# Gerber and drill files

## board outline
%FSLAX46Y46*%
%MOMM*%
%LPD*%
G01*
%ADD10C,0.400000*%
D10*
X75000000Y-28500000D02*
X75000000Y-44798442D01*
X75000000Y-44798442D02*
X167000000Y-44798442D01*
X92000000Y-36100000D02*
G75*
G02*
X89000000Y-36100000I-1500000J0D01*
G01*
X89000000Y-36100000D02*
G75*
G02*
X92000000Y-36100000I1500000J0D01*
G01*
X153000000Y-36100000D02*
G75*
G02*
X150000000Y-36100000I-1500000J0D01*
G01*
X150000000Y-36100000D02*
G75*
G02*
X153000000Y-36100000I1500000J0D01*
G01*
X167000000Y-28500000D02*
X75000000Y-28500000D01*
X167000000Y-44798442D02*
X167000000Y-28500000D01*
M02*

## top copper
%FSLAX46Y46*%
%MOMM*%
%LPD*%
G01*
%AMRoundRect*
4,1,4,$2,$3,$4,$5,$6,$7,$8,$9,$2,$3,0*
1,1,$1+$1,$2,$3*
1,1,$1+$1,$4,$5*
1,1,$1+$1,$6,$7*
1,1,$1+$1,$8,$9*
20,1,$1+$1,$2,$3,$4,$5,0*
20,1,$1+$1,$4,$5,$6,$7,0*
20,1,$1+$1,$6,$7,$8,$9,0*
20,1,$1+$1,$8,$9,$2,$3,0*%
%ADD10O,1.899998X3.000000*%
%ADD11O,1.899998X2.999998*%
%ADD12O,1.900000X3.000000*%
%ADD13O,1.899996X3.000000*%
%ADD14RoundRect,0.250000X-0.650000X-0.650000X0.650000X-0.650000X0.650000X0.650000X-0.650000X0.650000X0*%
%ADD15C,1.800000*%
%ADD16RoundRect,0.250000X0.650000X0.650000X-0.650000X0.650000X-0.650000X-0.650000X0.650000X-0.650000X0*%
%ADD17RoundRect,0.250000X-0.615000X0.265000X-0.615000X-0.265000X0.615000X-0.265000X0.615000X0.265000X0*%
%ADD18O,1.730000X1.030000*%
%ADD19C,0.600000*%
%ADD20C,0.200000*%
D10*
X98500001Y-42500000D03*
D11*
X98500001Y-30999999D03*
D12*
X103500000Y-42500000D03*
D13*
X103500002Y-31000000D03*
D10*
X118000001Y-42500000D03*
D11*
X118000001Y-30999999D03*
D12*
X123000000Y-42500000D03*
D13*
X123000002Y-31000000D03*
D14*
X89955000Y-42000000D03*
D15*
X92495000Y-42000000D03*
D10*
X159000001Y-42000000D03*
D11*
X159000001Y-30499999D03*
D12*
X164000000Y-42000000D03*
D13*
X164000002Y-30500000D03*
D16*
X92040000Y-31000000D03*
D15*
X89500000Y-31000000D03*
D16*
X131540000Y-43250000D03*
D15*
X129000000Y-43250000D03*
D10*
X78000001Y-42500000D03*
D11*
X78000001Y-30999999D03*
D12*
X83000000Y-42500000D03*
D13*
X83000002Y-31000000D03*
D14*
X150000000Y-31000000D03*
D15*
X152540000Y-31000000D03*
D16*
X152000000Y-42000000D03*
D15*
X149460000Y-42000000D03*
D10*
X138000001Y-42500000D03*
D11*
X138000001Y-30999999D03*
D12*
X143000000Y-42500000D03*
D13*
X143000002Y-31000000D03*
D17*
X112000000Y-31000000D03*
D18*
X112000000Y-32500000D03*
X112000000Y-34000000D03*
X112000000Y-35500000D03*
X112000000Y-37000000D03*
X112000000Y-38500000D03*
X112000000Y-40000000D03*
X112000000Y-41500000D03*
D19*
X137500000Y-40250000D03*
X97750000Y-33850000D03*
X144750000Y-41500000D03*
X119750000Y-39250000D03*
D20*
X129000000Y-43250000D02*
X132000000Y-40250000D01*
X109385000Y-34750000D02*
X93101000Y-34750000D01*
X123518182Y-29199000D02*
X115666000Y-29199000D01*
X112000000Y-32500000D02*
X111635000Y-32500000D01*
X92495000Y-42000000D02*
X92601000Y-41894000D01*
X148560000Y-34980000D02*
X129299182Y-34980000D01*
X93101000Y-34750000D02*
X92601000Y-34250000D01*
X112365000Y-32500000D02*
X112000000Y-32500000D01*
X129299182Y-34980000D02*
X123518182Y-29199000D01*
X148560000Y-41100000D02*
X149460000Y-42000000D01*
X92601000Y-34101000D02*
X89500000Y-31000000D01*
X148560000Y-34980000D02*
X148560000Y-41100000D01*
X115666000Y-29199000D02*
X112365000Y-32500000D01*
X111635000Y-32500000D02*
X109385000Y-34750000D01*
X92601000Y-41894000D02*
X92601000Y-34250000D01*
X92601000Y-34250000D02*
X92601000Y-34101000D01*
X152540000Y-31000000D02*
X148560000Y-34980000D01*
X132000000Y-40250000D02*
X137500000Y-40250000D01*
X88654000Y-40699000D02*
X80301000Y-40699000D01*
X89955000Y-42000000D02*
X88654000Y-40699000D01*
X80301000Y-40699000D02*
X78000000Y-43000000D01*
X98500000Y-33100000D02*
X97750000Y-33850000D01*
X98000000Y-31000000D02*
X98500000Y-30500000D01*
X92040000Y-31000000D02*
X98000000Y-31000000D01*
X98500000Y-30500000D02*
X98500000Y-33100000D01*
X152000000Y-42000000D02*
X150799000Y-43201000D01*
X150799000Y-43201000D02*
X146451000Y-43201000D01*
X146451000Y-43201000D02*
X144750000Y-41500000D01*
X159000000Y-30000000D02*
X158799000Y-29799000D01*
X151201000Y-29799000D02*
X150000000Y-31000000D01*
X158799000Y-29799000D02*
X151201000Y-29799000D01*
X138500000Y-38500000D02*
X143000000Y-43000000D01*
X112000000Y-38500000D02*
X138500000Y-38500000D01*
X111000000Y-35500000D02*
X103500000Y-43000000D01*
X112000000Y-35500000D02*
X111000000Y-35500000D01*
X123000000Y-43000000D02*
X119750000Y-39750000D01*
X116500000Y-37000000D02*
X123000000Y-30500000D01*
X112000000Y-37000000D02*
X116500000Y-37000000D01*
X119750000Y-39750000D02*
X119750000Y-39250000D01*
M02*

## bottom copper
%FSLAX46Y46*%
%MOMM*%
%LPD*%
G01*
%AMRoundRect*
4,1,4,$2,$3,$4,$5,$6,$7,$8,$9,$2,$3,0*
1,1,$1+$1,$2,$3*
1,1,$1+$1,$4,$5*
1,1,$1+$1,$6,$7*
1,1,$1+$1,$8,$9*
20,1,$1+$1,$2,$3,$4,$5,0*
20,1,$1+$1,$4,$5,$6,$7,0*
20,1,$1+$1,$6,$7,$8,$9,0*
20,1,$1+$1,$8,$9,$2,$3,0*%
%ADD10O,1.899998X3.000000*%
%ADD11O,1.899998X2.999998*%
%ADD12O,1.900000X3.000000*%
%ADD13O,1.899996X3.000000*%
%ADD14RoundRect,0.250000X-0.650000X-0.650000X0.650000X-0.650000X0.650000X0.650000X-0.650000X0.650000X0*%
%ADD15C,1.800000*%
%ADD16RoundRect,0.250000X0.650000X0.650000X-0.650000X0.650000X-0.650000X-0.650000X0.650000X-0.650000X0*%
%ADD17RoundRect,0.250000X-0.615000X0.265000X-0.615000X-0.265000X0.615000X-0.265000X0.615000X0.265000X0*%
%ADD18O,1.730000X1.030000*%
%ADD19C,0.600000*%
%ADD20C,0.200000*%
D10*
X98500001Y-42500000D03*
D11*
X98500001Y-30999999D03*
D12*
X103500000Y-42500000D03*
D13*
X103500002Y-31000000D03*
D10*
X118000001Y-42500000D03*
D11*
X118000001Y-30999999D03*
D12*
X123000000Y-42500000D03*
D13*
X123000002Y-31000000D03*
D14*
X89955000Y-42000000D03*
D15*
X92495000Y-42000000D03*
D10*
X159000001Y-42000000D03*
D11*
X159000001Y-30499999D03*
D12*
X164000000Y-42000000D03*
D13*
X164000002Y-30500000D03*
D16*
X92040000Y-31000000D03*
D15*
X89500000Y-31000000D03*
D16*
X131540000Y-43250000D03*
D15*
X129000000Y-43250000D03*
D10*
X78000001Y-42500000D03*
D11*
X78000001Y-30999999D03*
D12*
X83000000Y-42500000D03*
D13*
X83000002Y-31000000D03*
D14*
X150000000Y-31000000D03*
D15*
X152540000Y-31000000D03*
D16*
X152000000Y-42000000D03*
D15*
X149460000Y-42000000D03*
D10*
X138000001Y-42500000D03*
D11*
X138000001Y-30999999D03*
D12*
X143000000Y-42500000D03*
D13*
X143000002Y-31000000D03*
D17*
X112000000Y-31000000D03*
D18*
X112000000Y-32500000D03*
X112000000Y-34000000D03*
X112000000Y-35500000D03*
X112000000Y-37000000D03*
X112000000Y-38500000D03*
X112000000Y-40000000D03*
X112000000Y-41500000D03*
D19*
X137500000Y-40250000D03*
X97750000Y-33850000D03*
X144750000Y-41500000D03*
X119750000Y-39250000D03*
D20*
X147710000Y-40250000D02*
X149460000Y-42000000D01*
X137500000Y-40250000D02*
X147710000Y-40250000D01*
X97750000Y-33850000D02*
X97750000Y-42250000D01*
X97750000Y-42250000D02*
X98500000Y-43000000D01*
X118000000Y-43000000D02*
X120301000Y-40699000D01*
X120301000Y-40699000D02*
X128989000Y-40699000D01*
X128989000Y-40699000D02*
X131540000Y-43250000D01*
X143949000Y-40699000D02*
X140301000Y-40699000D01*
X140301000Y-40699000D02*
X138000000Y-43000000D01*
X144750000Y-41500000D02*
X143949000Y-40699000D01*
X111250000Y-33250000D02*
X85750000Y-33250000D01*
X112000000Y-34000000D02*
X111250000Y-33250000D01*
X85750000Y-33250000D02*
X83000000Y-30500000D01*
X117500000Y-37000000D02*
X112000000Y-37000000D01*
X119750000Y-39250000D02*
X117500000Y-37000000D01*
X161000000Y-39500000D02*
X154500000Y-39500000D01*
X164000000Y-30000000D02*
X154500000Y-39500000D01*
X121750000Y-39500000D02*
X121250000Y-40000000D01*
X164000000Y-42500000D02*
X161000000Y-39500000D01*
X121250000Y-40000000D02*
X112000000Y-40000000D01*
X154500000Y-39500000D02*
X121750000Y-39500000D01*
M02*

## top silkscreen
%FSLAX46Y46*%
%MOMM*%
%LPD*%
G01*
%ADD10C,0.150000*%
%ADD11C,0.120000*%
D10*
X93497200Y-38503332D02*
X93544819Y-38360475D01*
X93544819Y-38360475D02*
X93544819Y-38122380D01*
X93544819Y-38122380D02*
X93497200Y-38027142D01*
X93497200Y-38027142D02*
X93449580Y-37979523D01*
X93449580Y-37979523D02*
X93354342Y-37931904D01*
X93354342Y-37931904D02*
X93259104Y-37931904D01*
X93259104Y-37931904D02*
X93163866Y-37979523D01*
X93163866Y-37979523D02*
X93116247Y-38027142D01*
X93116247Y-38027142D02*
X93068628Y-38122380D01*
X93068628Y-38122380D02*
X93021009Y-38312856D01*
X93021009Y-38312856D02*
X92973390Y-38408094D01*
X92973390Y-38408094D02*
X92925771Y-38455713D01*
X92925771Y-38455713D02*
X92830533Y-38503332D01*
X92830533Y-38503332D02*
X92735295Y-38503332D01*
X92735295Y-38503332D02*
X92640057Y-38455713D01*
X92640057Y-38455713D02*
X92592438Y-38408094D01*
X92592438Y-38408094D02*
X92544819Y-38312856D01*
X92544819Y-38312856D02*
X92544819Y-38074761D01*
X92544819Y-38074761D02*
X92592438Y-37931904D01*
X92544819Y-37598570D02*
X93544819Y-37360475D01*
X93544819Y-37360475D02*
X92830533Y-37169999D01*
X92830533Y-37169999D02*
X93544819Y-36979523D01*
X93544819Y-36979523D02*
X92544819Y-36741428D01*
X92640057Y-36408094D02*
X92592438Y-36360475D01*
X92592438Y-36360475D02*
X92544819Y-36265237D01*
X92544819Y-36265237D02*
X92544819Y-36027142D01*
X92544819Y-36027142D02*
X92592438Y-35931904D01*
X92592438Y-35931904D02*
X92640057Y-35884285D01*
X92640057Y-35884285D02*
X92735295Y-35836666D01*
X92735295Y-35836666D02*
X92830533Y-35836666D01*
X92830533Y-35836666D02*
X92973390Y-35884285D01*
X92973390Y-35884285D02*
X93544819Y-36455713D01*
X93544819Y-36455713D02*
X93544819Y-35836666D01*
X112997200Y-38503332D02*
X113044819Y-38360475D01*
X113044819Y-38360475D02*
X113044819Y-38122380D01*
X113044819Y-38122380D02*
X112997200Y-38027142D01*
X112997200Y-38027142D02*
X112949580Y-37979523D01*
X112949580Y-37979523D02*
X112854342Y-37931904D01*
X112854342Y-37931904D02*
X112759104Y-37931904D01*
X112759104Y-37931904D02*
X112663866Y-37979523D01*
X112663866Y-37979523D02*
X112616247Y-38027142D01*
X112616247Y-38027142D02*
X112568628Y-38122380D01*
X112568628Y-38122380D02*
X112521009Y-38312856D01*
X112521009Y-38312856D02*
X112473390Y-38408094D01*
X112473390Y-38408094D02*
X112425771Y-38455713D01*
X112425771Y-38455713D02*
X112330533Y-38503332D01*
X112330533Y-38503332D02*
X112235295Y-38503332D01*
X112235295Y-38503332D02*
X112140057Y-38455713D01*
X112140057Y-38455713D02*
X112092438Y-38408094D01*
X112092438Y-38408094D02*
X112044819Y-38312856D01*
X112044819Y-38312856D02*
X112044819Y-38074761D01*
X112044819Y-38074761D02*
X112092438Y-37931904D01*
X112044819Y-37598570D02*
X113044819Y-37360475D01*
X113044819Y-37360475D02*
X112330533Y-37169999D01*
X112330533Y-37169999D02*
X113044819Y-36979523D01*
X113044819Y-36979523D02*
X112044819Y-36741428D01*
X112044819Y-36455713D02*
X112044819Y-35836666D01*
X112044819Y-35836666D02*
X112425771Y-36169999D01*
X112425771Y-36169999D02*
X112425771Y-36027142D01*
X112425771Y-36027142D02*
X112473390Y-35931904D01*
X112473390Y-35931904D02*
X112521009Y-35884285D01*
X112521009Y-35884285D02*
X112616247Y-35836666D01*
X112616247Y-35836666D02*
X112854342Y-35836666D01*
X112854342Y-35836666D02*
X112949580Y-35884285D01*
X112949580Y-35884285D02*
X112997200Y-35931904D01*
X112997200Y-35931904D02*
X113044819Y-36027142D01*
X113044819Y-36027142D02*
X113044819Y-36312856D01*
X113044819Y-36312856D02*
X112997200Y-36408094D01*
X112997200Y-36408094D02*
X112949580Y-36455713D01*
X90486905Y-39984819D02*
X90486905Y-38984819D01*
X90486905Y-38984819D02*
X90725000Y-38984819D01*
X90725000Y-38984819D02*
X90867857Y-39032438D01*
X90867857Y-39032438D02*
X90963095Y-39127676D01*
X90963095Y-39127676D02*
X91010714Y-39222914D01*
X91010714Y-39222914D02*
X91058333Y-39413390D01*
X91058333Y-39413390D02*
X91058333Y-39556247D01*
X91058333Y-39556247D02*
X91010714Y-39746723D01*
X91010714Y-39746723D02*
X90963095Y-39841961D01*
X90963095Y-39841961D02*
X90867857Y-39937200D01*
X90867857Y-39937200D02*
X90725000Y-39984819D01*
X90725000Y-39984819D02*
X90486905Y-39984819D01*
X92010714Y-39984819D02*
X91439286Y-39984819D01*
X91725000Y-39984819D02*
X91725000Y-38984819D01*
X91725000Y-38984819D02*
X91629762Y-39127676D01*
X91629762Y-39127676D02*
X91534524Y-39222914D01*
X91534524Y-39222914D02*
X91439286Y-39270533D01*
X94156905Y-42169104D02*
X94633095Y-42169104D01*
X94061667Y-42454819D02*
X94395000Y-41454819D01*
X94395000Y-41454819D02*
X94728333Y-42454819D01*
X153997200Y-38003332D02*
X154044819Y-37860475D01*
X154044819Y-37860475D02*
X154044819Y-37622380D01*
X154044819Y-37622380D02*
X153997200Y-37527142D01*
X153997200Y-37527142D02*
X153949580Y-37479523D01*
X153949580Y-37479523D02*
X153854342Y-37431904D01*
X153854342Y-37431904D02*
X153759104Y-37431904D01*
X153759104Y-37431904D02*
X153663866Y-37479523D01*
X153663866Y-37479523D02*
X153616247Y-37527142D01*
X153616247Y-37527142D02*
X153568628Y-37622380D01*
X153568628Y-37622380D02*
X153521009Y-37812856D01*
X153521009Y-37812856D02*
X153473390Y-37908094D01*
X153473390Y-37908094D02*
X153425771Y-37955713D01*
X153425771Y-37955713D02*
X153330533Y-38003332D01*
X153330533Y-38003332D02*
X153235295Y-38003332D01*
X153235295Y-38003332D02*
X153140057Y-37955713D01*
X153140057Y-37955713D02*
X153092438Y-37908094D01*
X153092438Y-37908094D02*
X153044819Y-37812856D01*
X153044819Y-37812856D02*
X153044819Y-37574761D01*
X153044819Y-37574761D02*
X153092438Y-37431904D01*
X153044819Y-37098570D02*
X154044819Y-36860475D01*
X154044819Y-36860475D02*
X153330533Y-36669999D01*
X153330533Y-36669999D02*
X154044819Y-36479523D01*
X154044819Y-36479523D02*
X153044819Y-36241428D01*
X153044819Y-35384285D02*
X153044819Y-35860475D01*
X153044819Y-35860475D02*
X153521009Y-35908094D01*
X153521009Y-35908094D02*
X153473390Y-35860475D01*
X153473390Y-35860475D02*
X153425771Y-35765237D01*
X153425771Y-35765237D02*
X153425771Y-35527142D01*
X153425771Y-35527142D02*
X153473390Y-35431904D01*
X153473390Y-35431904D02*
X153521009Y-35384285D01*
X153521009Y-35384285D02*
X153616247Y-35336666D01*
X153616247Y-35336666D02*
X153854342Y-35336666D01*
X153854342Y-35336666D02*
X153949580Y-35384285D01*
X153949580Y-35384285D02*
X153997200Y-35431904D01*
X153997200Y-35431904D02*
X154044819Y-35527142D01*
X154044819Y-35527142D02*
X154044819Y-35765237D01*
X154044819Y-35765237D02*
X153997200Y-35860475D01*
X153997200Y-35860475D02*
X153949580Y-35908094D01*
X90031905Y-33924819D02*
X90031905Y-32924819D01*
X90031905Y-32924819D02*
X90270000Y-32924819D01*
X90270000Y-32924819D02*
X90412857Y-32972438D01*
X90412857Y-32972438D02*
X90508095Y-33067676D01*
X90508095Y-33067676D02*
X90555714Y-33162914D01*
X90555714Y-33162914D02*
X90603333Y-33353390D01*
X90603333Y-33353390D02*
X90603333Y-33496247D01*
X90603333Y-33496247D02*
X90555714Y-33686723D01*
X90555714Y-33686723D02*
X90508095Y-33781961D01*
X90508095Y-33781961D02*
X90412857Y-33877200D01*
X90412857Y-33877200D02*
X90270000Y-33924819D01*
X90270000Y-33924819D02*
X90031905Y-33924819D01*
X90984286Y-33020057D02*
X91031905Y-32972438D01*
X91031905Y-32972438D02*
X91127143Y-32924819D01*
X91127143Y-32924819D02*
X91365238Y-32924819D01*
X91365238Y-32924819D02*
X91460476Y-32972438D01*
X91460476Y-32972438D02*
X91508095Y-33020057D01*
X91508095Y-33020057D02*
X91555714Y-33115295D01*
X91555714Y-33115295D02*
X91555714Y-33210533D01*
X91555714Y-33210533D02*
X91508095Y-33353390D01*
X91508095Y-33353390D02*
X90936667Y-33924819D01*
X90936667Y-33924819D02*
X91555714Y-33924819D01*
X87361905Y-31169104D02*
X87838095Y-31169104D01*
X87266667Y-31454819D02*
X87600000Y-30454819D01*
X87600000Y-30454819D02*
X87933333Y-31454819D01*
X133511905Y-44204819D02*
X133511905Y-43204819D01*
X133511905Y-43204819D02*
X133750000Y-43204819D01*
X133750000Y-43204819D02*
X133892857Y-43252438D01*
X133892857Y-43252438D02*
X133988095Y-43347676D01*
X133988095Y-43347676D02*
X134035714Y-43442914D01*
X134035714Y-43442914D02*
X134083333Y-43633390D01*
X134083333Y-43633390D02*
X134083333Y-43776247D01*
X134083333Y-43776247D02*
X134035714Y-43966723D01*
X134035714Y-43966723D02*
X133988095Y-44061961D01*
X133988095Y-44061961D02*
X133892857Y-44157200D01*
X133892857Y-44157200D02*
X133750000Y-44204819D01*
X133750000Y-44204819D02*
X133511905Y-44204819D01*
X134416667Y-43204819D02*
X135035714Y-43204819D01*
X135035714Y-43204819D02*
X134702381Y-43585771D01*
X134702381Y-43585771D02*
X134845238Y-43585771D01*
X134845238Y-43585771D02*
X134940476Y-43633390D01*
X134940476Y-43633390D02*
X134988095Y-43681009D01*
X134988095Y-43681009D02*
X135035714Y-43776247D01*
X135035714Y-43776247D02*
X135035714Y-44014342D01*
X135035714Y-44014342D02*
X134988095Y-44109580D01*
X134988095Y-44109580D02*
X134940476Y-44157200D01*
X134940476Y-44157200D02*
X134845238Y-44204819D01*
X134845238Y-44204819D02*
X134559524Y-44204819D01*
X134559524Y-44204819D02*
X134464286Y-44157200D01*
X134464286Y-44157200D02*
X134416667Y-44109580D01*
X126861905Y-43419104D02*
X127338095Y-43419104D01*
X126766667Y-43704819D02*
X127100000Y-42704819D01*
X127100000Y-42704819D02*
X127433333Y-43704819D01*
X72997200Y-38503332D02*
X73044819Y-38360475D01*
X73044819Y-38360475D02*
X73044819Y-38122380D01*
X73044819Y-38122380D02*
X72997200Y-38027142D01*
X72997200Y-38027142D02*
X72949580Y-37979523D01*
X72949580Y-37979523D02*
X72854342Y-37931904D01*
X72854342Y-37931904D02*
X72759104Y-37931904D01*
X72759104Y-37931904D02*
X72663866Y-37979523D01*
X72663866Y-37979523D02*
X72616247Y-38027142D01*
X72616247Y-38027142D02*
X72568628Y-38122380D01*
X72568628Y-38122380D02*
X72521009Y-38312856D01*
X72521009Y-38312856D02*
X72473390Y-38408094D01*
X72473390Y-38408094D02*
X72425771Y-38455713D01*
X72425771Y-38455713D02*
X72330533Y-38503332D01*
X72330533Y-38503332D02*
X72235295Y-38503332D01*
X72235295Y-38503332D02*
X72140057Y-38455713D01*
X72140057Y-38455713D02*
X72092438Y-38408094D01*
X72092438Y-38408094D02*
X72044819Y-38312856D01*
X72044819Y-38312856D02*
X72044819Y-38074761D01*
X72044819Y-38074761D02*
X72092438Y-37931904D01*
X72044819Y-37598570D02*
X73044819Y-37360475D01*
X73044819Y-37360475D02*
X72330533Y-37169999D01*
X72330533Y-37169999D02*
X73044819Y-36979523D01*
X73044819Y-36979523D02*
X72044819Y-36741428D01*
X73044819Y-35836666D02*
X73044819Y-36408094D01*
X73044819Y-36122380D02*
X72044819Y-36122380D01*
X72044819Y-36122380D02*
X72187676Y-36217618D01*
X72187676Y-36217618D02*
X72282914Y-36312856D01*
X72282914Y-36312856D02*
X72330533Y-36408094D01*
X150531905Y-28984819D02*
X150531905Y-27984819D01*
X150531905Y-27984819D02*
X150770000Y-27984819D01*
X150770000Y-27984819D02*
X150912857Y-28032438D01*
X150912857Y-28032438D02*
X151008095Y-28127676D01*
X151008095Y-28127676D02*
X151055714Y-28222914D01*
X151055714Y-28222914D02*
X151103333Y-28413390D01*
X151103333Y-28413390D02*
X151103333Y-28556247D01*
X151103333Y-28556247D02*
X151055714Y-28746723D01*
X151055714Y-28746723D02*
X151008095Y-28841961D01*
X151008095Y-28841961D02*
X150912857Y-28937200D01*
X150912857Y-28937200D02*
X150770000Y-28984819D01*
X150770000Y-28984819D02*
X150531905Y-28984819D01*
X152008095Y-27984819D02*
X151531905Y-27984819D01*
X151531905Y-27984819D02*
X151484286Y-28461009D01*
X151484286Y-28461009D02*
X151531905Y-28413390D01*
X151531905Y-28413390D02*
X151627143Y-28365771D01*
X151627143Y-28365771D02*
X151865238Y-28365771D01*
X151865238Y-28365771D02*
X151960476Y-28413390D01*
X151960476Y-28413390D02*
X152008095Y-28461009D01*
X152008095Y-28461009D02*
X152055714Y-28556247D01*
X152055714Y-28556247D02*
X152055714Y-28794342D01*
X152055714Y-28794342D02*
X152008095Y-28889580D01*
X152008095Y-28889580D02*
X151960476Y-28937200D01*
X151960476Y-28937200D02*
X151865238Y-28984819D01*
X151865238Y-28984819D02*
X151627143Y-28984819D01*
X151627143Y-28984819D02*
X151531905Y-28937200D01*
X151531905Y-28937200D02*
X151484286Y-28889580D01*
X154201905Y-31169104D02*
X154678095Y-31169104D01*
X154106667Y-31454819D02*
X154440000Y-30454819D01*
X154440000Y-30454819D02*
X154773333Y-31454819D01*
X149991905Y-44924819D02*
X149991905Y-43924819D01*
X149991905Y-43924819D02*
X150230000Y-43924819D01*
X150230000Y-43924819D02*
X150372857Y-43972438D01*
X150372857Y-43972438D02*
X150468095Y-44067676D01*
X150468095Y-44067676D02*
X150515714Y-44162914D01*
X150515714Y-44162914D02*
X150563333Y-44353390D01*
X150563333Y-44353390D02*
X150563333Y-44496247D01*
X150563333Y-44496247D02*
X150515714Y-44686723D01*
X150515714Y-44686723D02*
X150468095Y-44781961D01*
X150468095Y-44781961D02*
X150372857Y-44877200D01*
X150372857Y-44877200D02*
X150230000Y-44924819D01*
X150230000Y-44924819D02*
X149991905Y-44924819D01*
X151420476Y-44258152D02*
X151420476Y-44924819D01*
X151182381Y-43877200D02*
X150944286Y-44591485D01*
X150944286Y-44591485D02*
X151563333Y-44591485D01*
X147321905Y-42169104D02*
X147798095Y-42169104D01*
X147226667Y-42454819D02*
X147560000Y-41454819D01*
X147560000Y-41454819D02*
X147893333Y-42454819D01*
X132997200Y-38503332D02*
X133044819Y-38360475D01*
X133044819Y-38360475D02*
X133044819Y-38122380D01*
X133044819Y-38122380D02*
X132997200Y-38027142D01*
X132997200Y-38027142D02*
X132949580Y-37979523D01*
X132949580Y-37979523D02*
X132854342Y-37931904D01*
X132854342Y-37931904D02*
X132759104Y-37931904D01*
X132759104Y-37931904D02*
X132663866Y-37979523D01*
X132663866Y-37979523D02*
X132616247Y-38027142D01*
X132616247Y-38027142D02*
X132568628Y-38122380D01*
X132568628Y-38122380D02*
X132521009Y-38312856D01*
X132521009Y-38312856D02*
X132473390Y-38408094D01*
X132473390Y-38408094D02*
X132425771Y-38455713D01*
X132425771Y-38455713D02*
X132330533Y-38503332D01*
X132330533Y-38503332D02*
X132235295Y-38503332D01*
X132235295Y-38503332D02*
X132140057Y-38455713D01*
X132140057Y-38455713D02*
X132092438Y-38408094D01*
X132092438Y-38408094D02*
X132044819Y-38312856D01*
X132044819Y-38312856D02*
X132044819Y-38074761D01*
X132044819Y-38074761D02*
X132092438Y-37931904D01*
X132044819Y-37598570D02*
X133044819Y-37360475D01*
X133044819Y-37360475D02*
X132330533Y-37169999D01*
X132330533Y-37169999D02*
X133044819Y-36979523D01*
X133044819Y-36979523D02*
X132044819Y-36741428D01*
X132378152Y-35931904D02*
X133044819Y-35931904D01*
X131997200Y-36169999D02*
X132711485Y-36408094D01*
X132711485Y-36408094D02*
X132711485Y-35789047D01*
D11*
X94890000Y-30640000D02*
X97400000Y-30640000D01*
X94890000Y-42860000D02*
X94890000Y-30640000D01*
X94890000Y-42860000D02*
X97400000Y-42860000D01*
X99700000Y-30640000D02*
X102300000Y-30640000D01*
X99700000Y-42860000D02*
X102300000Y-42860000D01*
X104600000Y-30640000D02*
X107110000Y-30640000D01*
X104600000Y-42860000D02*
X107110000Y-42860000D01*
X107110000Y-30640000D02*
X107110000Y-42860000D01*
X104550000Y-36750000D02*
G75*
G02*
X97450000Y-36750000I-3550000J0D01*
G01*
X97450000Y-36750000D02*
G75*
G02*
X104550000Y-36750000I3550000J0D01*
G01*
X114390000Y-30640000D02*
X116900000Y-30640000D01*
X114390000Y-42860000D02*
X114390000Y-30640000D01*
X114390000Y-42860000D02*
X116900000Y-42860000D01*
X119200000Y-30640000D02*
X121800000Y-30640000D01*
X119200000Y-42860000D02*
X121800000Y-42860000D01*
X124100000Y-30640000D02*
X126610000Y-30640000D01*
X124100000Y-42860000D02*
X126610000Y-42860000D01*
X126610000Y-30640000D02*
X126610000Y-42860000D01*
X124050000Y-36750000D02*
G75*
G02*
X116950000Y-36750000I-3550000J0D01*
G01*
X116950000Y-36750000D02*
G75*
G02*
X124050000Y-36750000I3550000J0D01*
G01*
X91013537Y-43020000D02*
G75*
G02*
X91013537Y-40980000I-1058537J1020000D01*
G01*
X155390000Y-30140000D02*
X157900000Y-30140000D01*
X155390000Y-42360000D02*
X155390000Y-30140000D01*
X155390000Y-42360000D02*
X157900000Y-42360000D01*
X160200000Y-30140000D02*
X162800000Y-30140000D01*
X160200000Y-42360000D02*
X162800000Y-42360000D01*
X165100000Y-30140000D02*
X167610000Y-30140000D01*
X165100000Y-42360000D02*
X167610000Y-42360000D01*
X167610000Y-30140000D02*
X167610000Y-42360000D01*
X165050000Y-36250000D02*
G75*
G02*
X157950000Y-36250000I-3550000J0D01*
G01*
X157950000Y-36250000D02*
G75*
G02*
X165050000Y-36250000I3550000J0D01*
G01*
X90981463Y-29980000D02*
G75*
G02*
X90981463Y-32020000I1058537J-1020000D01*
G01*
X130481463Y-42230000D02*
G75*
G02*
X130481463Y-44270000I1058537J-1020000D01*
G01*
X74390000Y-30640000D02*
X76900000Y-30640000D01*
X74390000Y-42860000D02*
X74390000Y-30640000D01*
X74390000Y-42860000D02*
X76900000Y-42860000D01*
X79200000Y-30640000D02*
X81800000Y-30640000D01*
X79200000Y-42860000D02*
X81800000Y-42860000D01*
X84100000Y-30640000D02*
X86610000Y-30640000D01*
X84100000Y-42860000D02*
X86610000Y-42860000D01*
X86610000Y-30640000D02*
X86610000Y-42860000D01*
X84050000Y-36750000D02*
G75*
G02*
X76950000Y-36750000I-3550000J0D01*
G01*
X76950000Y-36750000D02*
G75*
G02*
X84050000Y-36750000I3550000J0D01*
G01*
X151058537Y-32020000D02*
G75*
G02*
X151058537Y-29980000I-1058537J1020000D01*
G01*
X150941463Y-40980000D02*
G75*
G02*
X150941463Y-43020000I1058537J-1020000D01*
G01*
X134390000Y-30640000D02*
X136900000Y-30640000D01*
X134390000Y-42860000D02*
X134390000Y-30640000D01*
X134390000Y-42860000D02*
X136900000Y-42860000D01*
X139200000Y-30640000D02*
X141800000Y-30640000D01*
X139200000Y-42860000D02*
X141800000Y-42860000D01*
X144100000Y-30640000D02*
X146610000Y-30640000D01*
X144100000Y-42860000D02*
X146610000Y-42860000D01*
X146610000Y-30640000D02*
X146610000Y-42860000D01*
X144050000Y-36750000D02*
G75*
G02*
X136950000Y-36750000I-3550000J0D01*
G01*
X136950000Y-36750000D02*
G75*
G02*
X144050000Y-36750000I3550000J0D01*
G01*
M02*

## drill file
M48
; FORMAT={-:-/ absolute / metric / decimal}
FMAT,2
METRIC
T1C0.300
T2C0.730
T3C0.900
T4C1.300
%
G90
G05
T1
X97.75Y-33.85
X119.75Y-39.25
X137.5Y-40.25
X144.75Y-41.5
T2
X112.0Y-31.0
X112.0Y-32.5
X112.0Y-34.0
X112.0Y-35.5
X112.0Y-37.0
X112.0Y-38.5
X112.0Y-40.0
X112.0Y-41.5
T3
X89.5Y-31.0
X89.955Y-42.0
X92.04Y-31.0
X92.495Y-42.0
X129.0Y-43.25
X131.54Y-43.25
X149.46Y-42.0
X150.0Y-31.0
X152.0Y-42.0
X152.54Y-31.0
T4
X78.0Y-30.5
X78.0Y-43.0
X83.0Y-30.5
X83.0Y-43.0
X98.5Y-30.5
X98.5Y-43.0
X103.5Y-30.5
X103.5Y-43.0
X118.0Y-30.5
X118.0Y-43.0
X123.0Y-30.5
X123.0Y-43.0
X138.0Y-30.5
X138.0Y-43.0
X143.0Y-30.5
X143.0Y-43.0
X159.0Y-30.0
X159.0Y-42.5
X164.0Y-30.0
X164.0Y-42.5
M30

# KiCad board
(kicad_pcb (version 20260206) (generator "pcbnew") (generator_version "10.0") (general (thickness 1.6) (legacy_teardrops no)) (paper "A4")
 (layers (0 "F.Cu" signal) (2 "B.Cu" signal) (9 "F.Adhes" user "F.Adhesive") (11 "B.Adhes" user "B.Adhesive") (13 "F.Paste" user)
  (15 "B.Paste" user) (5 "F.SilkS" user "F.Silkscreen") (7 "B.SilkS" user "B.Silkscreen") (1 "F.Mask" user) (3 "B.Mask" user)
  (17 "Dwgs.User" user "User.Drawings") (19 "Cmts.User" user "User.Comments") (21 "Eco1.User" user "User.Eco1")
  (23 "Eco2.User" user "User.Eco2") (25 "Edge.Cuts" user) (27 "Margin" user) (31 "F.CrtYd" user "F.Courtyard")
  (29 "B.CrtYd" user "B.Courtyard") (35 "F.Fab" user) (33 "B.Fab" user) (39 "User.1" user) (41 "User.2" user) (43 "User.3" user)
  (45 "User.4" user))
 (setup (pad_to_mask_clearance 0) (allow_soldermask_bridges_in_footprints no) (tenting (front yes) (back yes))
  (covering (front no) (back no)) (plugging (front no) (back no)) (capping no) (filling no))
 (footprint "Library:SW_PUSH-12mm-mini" (layer "F.Cu") (at 98.5 43 90)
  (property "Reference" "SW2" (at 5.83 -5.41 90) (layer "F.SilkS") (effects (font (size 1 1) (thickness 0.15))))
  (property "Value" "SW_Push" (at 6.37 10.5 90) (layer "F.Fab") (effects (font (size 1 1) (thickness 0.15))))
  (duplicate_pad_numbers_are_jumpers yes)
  (fp_line (start 12.36 -3.61) (end 12.36 -1.1) (stroke (width 0.12) (type default)) (layer "F.SilkS"))
  (fp_line (start 0.14 -3.61) (end 12.36 -3.61) (stroke (width 0.12) (type default)) (layer "F.SilkS"))
  (fp_line (start 0.14 -3.61) (end 0.14 -1.1) (stroke (width 0.12) (type default)) (layer "F.SilkS"))
  (fp_line (start 12.36 1.2) (end 12.36 3.8) (stroke (width 0.12) (type default)) (layer "F.SilkS"))
  (fp_line (start 0.14 1.2) (end 0.14 3.8) (stroke (width 0.12) (type default)) (layer "F.SilkS"))
  (fp_line (start 12.36 6.1) (end 12.36 8.61) (stroke (width 0.12) (type default)) (layer "F.SilkS"))
  (fp_line (start 0.14 6.1) (end 0.14 8.61) (stroke (width 0.12) (type default)) (layer "F.SilkS"))
  (fp_line (start 12.36 8.61) (end 0.14 8.61) (stroke (width 0.12) (type default)) (layer "F.SilkS"))
  (fp_circle (center 6.25 2.5) (end 9.8 2.5) (stroke (width 0.12) (type default)) (fill no) (layer "F.SilkS"))
  (pad "1" thru_hole oval (at 0 0 90) (size 3 1.899998) (drill 1.3 (offset 0.5 0.000001)) (layers "*.Cu" "*.Mask") (remove_unused_layers no)
   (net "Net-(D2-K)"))
  (pad "1" thru_hole oval (at 12.5 0 90) (size 2.999998 1.899998) (drill 1.3 (offset -0.499999 0.000001)) (layers "*.Cu" "*.Mask")
   (remove_unused_layers no) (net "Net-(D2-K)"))
  (pad "2" thru_hole oval (at 0 5 90) (size 3 1.9) (drill 1.3 (offset 0.5 0)) (layers "*.Cu" "*.Mask") (remove_unused_layers no)
   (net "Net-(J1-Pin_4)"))
  (pad "2" thru_hole oval (at 12.5 5 90) (size 3 1.899996) (drill 1.3 (offset -0.5 0.000002)) (layers "*.Cu" "*.Mask")
   (remove_unused_layers no) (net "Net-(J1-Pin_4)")))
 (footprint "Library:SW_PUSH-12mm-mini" (layer "F.Cu") (at 118 43 90)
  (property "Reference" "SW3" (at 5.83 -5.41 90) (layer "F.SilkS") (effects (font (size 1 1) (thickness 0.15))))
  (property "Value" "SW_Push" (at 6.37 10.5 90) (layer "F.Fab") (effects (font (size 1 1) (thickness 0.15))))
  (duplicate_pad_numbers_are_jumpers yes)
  (fp_line (start 12.36 -3.61) (end 12.36 -1.1) (stroke (width 0.12) (type default)) (layer "F.SilkS"))
  (fp_line (start 0.14 -3.61) (end 12.36 -3.61) (stroke (width 0.12) (type default)) (layer "F.SilkS"))
  (fp_line (start 0.14 -3.61) (end 0.14 -1.1) (stroke (width 0.12) (type default)) (layer "F.SilkS"))
  (fp_line (start 12.36 1.2) (end 12.36 3.8) (stroke (width 0.12) (type default)) (layer "F.SilkS"))
  (fp_line (start 0.14 1.2) (end 0.14 3.8) (stroke (width 0.12) (type default)) (layer "F.SilkS"))
  (fp_line (start 12.36 6.1) (end 12.36 8.61) (stroke (width 0.12) (type default)) (layer "F.SilkS"))
  (fp_line (start 0.14 6.1) (end 0.14 8.61) (stroke (width 0.12) (type default)) (layer "F.SilkS"))
  (fp_line (start 12.36 8.61) (end 0.14 8.61) (stroke (width 0.12) (type default)) (layer "F.SilkS"))
  (fp_circle (center 6.25 2.5) (end 9.8 2.5) (stroke (width 0.12) (type default)) (fill no) (layer "F.SilkS"))
  (pad "1" thru_hole oval (at 0 0 90) (size 3 1.899998) (drill 1.3 (offset 0.5 0.000001)) (layers "*.Cu" "*.Mask") (remove_unused_layers no)
   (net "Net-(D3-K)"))
  (pad "1" thru_hole oval (at 12.5 0 90) (size 2.999998 1.899998) (drill 1.3 (offset -0.499999 0.000001)) (layers "*.Cu" "*.Mask")
   (remove_unused_layers no) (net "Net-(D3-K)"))
  (pad "2" thru_hole oval (at 0 5 90) (size 3 1.9) (drill 1.3 (offset 0.5 0)) (layers "*.Cu" "*.Mask") (remove_unused_layers no)
   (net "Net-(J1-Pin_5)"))
  (pad "2" thru_hole oval (at 12.5 5 90) (size 3 1.899996) (drill 1.3 (offset -0.5 0.000002)) (layers "*.Cu" "*.Mask")
   (remove_unused_layers no) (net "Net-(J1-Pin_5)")))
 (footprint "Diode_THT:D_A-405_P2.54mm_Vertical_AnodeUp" (layer "F.Cu") (at 89.955 42)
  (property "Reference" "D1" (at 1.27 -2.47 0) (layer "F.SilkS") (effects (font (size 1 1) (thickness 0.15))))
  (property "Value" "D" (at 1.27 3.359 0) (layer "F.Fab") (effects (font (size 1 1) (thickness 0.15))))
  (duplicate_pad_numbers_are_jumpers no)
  (fp_arc (start 1.058537 1.02) (mid -1.47 0) (end 1.058537 -1.02) (stroke (width 0.12) (type solid)) (layer "F.SilkS"))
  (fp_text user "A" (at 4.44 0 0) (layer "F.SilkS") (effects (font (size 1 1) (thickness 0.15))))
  (pad "1" thru_hole roundrect (at 0 0) (size 1.8 1.8) (drill 0.9) (layers "*.Cu" "*.Mask") (remove_unused_layers no)
   (roundrect_rratio 0.138889) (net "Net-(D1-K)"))
  (pad "2" thru_hole circle (at 2.54 0) (size 1.8 1.8) (drill 0.9) (layers "*.Cu" "*.Mask") (remove_unused_layers no) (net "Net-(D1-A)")))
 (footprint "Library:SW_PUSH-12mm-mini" (layer "F.Cu") (at 159 42.5 90)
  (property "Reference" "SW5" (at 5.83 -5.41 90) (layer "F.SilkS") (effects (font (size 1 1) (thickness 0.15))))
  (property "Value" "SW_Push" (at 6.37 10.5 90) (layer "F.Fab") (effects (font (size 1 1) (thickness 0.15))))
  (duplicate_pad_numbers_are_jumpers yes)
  (fp_line (start 12.36 -3.61) (end 12.36 -1.1) (stroke (width 0.12) (type default)) (layer "F.SilkS"))
  (fp_line (start 0.14 -3.61) (end 12.36 -3.61) (stroke (width 0.12) (type default)) (layer "F.SilkS"))
  (fp_line (start 0.14 -3.61) (end 0.14 -1.1) (stroke (width 0.12) (type default)) (layer "F.SilkS"))
  (fp_line (start 12.36 1.2) (end 12.36 3.8) (stroke (width 0.12) (type default)) (layer "F.SilkS"))
  (fp_line (start 0.14 1.2) (end 0.14 3.8) (stroke (width 0.12) (type default)) (layer "F.SilkS"))
  (fp_line (start 12.36 6.1) (end 12.36 8.61) (stroke (width 0.12) (type default)) (layer "F.SilkS"))
  (fp_line (start 0.14 6.1) (end 0.14 8.61) (stroke (width 0.12) (type default)) (layer "F.SilkS"))
  (fp_line (start 12.36 8.61) (end 0.14 8.61) (stroke (width 0.12) (type default)) (layer "F.SilkS"))
  (fp_circle (center 6.25 2.5) (end 9.8 2.5) (stroke (width 0.12) (type default)) (fill no) (layer "F.SilkS"))
  (pad "1" thru_hole oval (at 0 0 90) (size 3 1.899998) (drill 1.3 (offset 0.5 0.000001)) (layers "*.Cu" "*.Mask") (remove_unused_layers no)
   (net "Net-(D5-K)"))
  (pad "1" thru_hole oval (at 12.5 0 90) (size 2.999998 1.899998) (drill 1.3 (offset -0.499999 0.000001)) (layers "*.Cu" "*.Mask")
   (remove_unused_layers no) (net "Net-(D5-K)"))
  (pad "2" thru_hole oval (at 0 5 90) (size 3 1.9) (drill 1.3 (offset 0.5 0)) (layers "*.Cu" "*.Mask") (remove_unused_layers no)
   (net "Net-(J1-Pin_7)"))
  (pad "2" thru_hole oval (at 12.5 5 90) (size 3 1.899996) (drill 1.3 (offset -0.5 0.000002)) (layers "*.Cu" "*.Mask")
   (remove_unused_layers no) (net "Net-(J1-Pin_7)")))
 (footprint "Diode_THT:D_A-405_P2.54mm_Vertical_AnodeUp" (layer "F.Cu") (at 92.04 31 180)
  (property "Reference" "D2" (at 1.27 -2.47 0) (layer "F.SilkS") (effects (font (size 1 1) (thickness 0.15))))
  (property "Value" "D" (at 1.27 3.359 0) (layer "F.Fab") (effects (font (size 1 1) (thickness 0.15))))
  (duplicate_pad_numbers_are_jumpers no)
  (fp_arc (start 1.058537 1.02) (mid -1.47 0) (end 1.058537 -1.02) (stroke (width 0.12) (type solid)) (layer "F.SilkS"))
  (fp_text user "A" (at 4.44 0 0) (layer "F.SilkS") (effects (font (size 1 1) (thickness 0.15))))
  (pad "1" thru_hole roundrect (at 0 0 180) (size 1.8 1.8) (drill 0.9) (layers "*.Cu" "*.Mask") (remove_unused_layers no)
   (roundrect_rratio 0.138889) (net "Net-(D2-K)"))
  (pad "2" thru_hole circle (at 2.54 0 180) (size 1.8 1.8) (drill 0.9) (layers "*.Cu" "*.Mask") (remove_unused_layers no) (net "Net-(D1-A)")))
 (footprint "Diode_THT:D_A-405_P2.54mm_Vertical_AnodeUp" (layer "F.Cu") (at 131.54 43.25 180)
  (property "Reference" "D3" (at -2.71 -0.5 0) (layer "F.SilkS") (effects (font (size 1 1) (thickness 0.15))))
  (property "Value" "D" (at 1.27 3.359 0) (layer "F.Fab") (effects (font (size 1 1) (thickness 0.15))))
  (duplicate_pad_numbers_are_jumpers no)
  (fp_arc (start 1.058537 1.02) (mid -1.47 0) (end 1.058537 -1.02) (stroke (width 0.12) (type solid)) (layer "F.SilkS"))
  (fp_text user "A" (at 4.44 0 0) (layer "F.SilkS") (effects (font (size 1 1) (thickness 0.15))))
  (pad "1" thru_hole roundrect (at 0 0 180) (size 1.8 1.8) (drill 0.9) (layers "*.Cu" "*.Mask") (remove_unused_layers no)
   (roundrect_rratio 0.138889) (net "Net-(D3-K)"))
  (pad "2" thru_hole circle (at 2.54 0 180) (size 1.8 1.8) (drill 0.9) (layers "*.Cu" "*.Mask") (remove_unused_layers no) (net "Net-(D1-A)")))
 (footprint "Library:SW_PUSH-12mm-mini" (layer "F.Cu") (at 78 43 90)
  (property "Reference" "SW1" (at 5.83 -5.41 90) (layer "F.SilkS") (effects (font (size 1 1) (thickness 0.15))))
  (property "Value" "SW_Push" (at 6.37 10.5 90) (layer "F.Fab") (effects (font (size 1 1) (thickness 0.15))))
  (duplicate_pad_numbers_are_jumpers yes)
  (fp_line (start 12.36 -3.61) (end 12.36 -1.1) (stroke (width 0.12) (type default)) (layer "F.SilkS"))
  (fp_line (start 0.14 -3.61) (end 12.36 -3.61) (stroke (width 0.12) (type default)) (layer "F.SilkS"))
  (fp_line (start 0.14 -3.61) (end 0.14 -1.1) (stroke (width 0.12) (type default)) (layer "F.SilkS"))
  (fp_line (start 12.36 1.2) (end 12.36 3.8) (stroke (width 0.12) (type default)) (layer "F.SilkS"))
  (fp_line (start 0.14 1.2) (end 0.14 3.8) (stroke (width 0.12) (type default)) (layer "F.SilkS"))
  (fp_line (start 12.36 6.1) (end 12.36 8.61) (stroke (width 0.12) (type default)) (layer "F.SilkS"))
  (fp_line (start 0.14 6.1) (end 0.14 8.61) (stroke (width 0.12) (type default)) (layer "F.SilkS"))
  (fp_line (start 12.36 8.61) (end 0.14 8.61) (stroke (width 0.12) (type default)) (layer "F.SilkS"))
  (fp_circle (center 6.25 2.5) (end 9.8 2.5) (stroke (width 0.12) (type default)) (fill no) (layer "F.SilkS"))
  (pad "1" thru_hole oval (at 0 0 90) (size 3 1.899998) (drill 1.3 (offset 0.5 0.000001)) (layers "*.Cu" "*.Mask") (remove_unused_layers no)
   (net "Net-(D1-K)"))
  (pad "1" thru_hole oval (at 12.5 0 90) (size 2.999998 1.899998) (drill 1.3 (offset -0.499999 0.000001)) (layers "*.Cu" "*.Mask")
   (remove_unused_layers no) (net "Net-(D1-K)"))
  (pad "2" thru_hole oval (at 0 5 90) (size 3 1.9) (drill 1.3 (offset 0.5 0)) (layers "*.Cu" "*.Mask") (remove_unused_layers no)
   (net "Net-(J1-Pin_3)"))
  (pad "2" thru_hole oval (at 12.5 5 90) (size 3 1.899996) (drill 1.3 (offset -0.5 0.000002)) (layers "*.Cu" "*.Mask")
   (remove_unused_layers no) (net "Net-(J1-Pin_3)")))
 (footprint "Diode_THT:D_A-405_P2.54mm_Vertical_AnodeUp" (layer "F.Cu") (at 150 31)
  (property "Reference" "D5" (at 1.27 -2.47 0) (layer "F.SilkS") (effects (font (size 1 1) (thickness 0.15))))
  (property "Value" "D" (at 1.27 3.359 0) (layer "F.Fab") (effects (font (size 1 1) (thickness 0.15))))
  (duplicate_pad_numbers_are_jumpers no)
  (fp_arc (start 1.058537 1.02) (mid -1.47 0) (end 1.058537 -1.02) (stroke (width 0.12) (type solid)) (layer "F.SilkS"))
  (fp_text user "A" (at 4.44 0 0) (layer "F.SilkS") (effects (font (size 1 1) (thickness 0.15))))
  (pad "1" thru_hole roundrect (at 0 0) (size 1.8 1.8) (drill 0.9) (layers "*.Cu" "*.Mask") (remove_unused_layers no)
   (roundrect_rratio 0.138889) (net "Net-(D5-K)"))
  (pad "2" thru_hole circle (at 2.54 0) (size 1.8 1.8) (drill 0.9) (layers "*.Cu" "*.Mask") (remove_unused_layers no) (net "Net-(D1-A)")))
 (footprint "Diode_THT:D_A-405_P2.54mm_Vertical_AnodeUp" (layer "F.Cu") (at 152 42 180)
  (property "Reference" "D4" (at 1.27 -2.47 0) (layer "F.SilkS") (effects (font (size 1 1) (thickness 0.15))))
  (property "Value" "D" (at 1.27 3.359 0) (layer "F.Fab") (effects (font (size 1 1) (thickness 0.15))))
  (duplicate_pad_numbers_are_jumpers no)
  (fp_arc (start 1.058537 1.02) (mid -1.47 0) (end 1.058537 -1.02) (stroke (width 0.12) (type solid)) (layer "F.SilkS"))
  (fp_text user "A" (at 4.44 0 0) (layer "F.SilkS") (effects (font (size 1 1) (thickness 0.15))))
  (pad "1" thru_hole roundrect (at 0 0 180) (size 1.8 1.8) (drill 0.9) (layers "*.Cu" "*.Mask") (remove_unused_layers no)
   (roundrect_rratio 0.138889) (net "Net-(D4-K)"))
  (pad "2" thru_hole circle (at 2.54 0 180) (size 1.8 1.8) (drill 0.9) (layers "*.Cu" "*.Mask") (remove_unused_layers no) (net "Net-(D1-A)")))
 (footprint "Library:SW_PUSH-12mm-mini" (layer "F.Cu") (at 138 43 90)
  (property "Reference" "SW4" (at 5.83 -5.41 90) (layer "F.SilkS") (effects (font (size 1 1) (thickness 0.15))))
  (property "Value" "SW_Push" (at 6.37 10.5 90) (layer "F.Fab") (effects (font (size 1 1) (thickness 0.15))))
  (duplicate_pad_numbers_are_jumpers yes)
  (fp_line (start 12.36 -3.61) (end 12.36 -1.1) (stroke (width 0.12) (type default)) (layer "F.SilkS"))
  (fp_line (start 0.14 -3.61) (end 12.36 -3.61) (stroke (width 0.12) (type default)) (layer "F.SilkS"))
  (fp_line (start 0.14 -3.61) (end 0.14 -1.1) (stroke (width 0.12) (type default)) (layer "F.SilkS"))
  (fp_line (start 12.36 1.2) (end 12.36 3.8) (stroke (width 0.12) (type default)) (layer "F.SilkS"))
  (fp_line (start 0.14 1.2) (end 0.14 3.8) (stroke (width 0.12) (type default)) (layer "F.SilkS"))
  (fp_line (start 12.36 6.1) (end 12.36 8.61) (stroke (width 0.12) (type default)) (layer "F.SilkS"))
  (fp_line (start 0.14 6.1) (end 0.14 8.61) (stroke (width 0.12) (type default)) (layer "F.SilkS"))
  (fp_line (start 12.36 8.61) (end 0.14 8.61) (stroke (width 0.12) (type default)) (layer "F.SilkS"))
  (fp_circle (center 6.25 2.5) (end 9.8 2.5) (stroke (width 0.12) (type default)) (fill no) (layer "F.SilkS"))
  (pad "1" thru_hole oval (at 0 0 90) (size 3 1.899998) (drill 1.3 (offset 0.5 0.000001)) (layers "*.Cu" "*.Mask") (remove_unused_layers no)
   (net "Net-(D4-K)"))
  (pad "1" thru_hole oval (at 12.5 0 90) (size 2.999998 1.899998) (drill 1.3 (offset -0.499999 0.000001)) (layers "*.Cu" "*.Mask")
   (remove_unused_layers no) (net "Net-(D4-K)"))
  (pad "2" thru_hole oval (at 0 5 90) (size 3 1.9) (drill 1.3 (offset 0.5 0)) (layers "*.Cu" "*.Mask") (remove_unused_layers no)
   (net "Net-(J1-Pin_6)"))
  (pad "2" thru_hole oval (at 12.5 5 90) (size 3 1.899996) (drill 1.3 (offset -0.5 0.000002)) (layers "*.Cu" "*.Mask")
   (remove_unused_layers no) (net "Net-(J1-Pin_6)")))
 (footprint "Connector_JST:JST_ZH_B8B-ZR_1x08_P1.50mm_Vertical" (layer "B.Cu") (at 112 31 -90)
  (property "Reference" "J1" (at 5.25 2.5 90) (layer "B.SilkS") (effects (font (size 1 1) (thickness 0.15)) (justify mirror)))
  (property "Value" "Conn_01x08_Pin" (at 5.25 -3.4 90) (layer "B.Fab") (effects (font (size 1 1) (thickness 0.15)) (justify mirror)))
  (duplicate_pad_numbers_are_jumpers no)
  (pad "1" thru_hole roundrect (at 0 0 270) (size 1.03 1.73) (drill 0.73) (layers "*.Cu" "*.Mask") (remove_unused_layers no)
   (roundrect_rratio 0.242718) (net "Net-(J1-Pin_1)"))
  (pad "2" thru_hole oval (at 1.5 0 270) (size 1.03 1.73) (drill 0.73) (layers "*.Cu" "*.Mask") (remove_unused_layers no) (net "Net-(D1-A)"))
  (pad "3" thru_hole oval (at 3 0 270) (size 1.03 1.73) (drill 0.73) (layers "*.Cu" "*.Mask") (remove_unused_layers no)
   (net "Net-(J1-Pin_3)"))
  (pad "4" thru_hole oval (at 4.5 0 270) (size 1.03 1.73) (drill 0.73) (layers "*.Cu" "*.Mask") (remove_unused_layers no)
   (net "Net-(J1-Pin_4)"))
  (pad "5" thru_hole oval (at 6 0 270) (size 1.03 1.73) (drill 0.73) (layers "*.Cu" "*.Mask") (remove_unused_layers no)
   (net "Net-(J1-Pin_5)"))
  (pad "6" thru_hole oval (at 7.5 0 270) (size 1.03 1.73) (drill 0.73) (layers "*.Cu" "*.Mask") (remove_unused_layers no)
   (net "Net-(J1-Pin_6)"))
  (pad "7" thru_hole oval (at 9 0 270) (size 1.03 1.73) (drill 0.73) (layers "*.Cu" "*.Mask") (remove_unused_layers no)
   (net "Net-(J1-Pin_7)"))
  (pad "8" thru_hole oval (at 10.5 0 270) (size 1.03 1.73) (drill 0.73) (layers "*.Cu" "*.Mask") (remove_unused_layers no)
   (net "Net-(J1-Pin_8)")))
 (gr_line (start 75 28.5) (end 75 44.798442) (stroke (width 0.4) (type default)) (layer "Edge.Cuts"))
 (gr_line (start 75 44.798442) (end 167 44.798442) (stroke (width 0.4) (type default)) (layer "Edge.Cuts"))
 (gr_circle (center 90.5 36.1) (end 92 36.1) (stroke (width 0.4) (type default)) (fill no) (layer "Edge.Cuts"))
 (gr_circle (center 151.5 36.1) (end 153 36.1) (stroke (width 0.4) (type default)) (fill no) (layer "Edge.Cuts"))
 (gr_line (start 167 28.5) (end 75 28.5) (stroke (width 0.4) (type default)) (layer "Edge.Cuts"))
 (gr_line (start 167 44.798442) (end 167 28.5) (stroke (width 0.4) (type default)) (layer "Edge.Cuts"))
 (segment (start 129 43.25) (end 132 40.25) (width 0.2) (layer "F.Cu") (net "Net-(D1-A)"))
 (segment (start 109.385 34.75) (end 93.101 34.75) (width 0.2) (layer "F.Cu") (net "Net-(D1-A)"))
 (segment (start 123.518182 29.199) (end 115.666 29.199) (width 0.2) (layer "F.Cu") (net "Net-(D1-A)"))
 (segment (start 112 32.5) (end 111.635 32.5) (width 0.2) (layer "F.Cu") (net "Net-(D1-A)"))
 (segment (start 92.495 42) (end 92.601 41.894) (width 0.2) (layer "F.Cu") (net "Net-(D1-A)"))
 (segment (start 148.56 34.98) (end 129.299182 34.98) (width 0.2) (layer "F.Cu") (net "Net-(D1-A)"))
 (segment (start 93.101 34.75) (end 92.601 34.25) (width 0.2) (layer "F.Cu") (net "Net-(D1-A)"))
 (segment (start 112.365 32.5) (end 112 32.5) (width 0.2) (layer "F.Cu") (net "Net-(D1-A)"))
 (segment (start 129.299182 34.98) (end 123.518182 29.199) (width 0.2) (layer "F.Cu") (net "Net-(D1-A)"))
 (segment (start 148.56 41.1) (end 149.46 42) (width 0.2) (layer "F.Cu") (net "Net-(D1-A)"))
 (segment (start 92.601 34.101) (end 89.5 31) (width 0.2) (layer "F.Cu") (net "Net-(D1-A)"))
 (segment (start 148.56 34.98) (end 148.56 41.1) (width 0.2) (layer "F.Cu") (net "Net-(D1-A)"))
 (segment (start 115.666 29.199) (end 112.365 32.5) (width 0.2) (layer "F.Cu") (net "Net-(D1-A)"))
 (segment (start 111.635 32.5) (end 109.385 34.75) (width 0.2) (layer "F.Cu") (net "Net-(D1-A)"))
 (segment (start 92.601 41.894) (end 92.601 34.25) (width 0.2) (layer "F.Cu") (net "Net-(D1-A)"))
 (segment (start 92.601 34.25) (end 92.601 34.101) (width 0.2) (layer "F.Cu") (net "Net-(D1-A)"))
 (segment (start 152.54 31) (end 148.56 34.98) (width 0.2) (layer "F.Cu") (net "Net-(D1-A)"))
 (segment (start 132 40.25) (end 137.5 40.25) (width 0.2) (layer "F.Cu") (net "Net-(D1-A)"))
 (via (at 137.5 40.25) (size 0.6) (drill 0.3) (layers "F.Cu" "B.Cu") (capping no) (covering (front no) (back no))
  (plugging (front no) (back no)) (filling no) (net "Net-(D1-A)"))
 (segment (start 147.71 40.25) (end 149.46 42) (width 0.2) (layer "B.Cu") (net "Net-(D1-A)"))
 (segment (start 137.5 40.25) (end 147.71 40.25) (width 0.2) (layer "B.Cu") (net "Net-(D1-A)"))
 (segment (start 88.654 40.699) (end 80.301 40.699) (width 0.2) (layer "F.Cu") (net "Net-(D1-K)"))
 (segment (start 89.955 42) (end 88.654 40.699) (width 0.2) (layer "F.Cu") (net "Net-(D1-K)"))
 (segment (start 80.301 40.699) (end 78 43) (width 0.2) (layer "F.Cu") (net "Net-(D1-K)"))
 (segment (start 98.5 33.1) (end 97.75 33.85) (width 0.2) (layer "F.Cu") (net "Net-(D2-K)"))
 (segment (start 98 31) (end 98.5 30.5) (width 0.2) (layer "F.Cu") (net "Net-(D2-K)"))
 (segment (start 92.04 31) (end 98 31) (width 0.2) (layer "F.Cu") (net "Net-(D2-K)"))
 (segment (start 98.5 30.5) (end 98.5 33.1) (width 0.2) (layer "F.Cu") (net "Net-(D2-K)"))
 (via (at 97.75 33.85) (size 0.6) (drill 0.3) (layers "F.Cu" "B.Cu") (capping no) (covering (front no) (back no))
  (plugging (front no) (back no)) (filling no) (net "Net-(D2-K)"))
 (segment (start 97.75 33.85) (end 97.75 42.25) (width 0.2) (layer "B.Cu") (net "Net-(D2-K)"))
 (segment (start 97.75 42.25) (end 98.5 43) (width 0.2) (layer "B.Cu") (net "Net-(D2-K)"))
 (segment (start 118 43) (end 120.301 40.699) (width 0.2) (layer "B.Cu") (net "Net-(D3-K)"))
 (segment (start 120.301 40.699) (end 128.989 40.699) (width 0.2) (layer "B.Cu") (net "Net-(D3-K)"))
 (segment (start 128.989 40.699) (end 131.54 43.25) (width 0.2) (layer "B.Cu") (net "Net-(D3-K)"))
 (segment (start 152 42) (end 150.799 43.201) (width 0.2) (layer "F.Cu") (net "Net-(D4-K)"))
 (segment (start 150.799 43.201) (end 146.451 43.201) (width 0.2) (layer "F.Cu") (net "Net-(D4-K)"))
 (segment (start 146.451 43.201) (end 144.75 41.5) (width 0.2) (layer "F.Cu") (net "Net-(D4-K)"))
 (via (at 144.75 41.5) (size 0.6) (drill 0.3) (layers "F.Cu" "B.Cu") (capping no) (covering (front no) (back no))
  (plugging (front no) (back no)) (filling no) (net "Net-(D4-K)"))
 (segment (start 143.949 40.699) (end 140.301 40.699) (width 0.2) (layer "B.Cu") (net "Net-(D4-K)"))
 (segment (start 140.301 40.699) (end 138 43) (width 0.2) (layer "B.Cu") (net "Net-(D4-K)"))
 (segment (start 144.75 41.5) (end 143.949 40.699) (width 0.2) (layer "B.Cu") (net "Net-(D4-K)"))
 (segment (start 159 30) (end 158.799 29.799) (width 0.2) (layer "F.Cu") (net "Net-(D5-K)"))
 (segment (start 151.201 29.799) (end 150 31) (width 0.2) (layer "F.Cu") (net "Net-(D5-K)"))
 (segment (start 158.799 29.799) (end 151.201 29.799) (width 0.2) (layer "F.Cu") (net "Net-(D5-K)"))
 (segment (start 138.5 38.5) (end 143 43) (width 0.2) (layer "F.Cu") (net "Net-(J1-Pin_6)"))
 (segment (start 112 38.5) (end 138.5 38.5) (width 0.2) (layer "F.Cu") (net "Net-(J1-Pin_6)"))
 (segment (start 111.25 33.25) (end 85.75 33.25) (width 0.2) (layer "B.Cu") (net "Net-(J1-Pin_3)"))
 (segment (start 112 34) (end 111.25 33.25) (width 0.2) (layer "B.Cu") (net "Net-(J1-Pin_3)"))
 (segment (start 85.75 33.25) (end 83 30.5) (width 0.2) (layer "B.Cu") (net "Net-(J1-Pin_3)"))
 (segment (start 111 35.5) (end 103.5 43) (width 0.2) (layer "F.Cu") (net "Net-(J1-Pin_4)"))
 (segment (start 112 35.5) (end 111 35.5) (width 0.2) (layer "F.Cu") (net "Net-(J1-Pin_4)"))
 (segment (start 123 43) (end 119.75 39.75) (width 0.2) (layer "F.Cu") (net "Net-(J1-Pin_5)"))
 (segment (start 116.5 37) (end 123 30.5) (width 0.2) (layer "F.Cu") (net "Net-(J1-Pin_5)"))
 (segment (start 112 37) (end 116.5 37) (width 0.2) (layer "F.Cu") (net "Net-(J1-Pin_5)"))
 (segment (start 119.75 39.75) (end 119.75 39.25) (width 0.2) (layer "F.Cu") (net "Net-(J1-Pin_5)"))
 (via (at 119.75 39.25) (size 0.6) (drill 0.3) (layers "F.Cu" "B.Cu") (capping no) (covering (front no) (back no))
  (plugging (front no) (back no)) (filling no) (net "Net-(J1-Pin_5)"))
 (segment (start 117.5 37) (end 112 37) (width 0.2) (layer "B.Cu") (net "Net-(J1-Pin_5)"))
 (segment (start 119.75 39.25) (end 117.5 37) (width 0.2) (layer "B.Cu") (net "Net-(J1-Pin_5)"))
 (segment (start 161 39.5) (end 154.5 39.5) (width 0.2) (layer "B.Cu") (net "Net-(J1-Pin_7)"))
 (segment (start 164 30) (end 154.5 39.5) (width 0.2) (layer "B.Cu") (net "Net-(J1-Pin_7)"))
 (segment (start 121.75 39.5) (end 121.25 40) (width 0.2) (layer "B.Cu") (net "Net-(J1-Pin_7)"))
 (segment (start 164 42.5) (end 161 39.5) (width 0.2) (layer "B.Cu") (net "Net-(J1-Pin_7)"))
 (segment (start 121.25 40) (end 112 40) (width 0.2) (layer "B.Cu") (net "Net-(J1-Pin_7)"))
 (segment (start 154.5 39.5) (end 121.75 39.5) (width 0.2) (layer "B.Cu") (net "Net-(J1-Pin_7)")))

